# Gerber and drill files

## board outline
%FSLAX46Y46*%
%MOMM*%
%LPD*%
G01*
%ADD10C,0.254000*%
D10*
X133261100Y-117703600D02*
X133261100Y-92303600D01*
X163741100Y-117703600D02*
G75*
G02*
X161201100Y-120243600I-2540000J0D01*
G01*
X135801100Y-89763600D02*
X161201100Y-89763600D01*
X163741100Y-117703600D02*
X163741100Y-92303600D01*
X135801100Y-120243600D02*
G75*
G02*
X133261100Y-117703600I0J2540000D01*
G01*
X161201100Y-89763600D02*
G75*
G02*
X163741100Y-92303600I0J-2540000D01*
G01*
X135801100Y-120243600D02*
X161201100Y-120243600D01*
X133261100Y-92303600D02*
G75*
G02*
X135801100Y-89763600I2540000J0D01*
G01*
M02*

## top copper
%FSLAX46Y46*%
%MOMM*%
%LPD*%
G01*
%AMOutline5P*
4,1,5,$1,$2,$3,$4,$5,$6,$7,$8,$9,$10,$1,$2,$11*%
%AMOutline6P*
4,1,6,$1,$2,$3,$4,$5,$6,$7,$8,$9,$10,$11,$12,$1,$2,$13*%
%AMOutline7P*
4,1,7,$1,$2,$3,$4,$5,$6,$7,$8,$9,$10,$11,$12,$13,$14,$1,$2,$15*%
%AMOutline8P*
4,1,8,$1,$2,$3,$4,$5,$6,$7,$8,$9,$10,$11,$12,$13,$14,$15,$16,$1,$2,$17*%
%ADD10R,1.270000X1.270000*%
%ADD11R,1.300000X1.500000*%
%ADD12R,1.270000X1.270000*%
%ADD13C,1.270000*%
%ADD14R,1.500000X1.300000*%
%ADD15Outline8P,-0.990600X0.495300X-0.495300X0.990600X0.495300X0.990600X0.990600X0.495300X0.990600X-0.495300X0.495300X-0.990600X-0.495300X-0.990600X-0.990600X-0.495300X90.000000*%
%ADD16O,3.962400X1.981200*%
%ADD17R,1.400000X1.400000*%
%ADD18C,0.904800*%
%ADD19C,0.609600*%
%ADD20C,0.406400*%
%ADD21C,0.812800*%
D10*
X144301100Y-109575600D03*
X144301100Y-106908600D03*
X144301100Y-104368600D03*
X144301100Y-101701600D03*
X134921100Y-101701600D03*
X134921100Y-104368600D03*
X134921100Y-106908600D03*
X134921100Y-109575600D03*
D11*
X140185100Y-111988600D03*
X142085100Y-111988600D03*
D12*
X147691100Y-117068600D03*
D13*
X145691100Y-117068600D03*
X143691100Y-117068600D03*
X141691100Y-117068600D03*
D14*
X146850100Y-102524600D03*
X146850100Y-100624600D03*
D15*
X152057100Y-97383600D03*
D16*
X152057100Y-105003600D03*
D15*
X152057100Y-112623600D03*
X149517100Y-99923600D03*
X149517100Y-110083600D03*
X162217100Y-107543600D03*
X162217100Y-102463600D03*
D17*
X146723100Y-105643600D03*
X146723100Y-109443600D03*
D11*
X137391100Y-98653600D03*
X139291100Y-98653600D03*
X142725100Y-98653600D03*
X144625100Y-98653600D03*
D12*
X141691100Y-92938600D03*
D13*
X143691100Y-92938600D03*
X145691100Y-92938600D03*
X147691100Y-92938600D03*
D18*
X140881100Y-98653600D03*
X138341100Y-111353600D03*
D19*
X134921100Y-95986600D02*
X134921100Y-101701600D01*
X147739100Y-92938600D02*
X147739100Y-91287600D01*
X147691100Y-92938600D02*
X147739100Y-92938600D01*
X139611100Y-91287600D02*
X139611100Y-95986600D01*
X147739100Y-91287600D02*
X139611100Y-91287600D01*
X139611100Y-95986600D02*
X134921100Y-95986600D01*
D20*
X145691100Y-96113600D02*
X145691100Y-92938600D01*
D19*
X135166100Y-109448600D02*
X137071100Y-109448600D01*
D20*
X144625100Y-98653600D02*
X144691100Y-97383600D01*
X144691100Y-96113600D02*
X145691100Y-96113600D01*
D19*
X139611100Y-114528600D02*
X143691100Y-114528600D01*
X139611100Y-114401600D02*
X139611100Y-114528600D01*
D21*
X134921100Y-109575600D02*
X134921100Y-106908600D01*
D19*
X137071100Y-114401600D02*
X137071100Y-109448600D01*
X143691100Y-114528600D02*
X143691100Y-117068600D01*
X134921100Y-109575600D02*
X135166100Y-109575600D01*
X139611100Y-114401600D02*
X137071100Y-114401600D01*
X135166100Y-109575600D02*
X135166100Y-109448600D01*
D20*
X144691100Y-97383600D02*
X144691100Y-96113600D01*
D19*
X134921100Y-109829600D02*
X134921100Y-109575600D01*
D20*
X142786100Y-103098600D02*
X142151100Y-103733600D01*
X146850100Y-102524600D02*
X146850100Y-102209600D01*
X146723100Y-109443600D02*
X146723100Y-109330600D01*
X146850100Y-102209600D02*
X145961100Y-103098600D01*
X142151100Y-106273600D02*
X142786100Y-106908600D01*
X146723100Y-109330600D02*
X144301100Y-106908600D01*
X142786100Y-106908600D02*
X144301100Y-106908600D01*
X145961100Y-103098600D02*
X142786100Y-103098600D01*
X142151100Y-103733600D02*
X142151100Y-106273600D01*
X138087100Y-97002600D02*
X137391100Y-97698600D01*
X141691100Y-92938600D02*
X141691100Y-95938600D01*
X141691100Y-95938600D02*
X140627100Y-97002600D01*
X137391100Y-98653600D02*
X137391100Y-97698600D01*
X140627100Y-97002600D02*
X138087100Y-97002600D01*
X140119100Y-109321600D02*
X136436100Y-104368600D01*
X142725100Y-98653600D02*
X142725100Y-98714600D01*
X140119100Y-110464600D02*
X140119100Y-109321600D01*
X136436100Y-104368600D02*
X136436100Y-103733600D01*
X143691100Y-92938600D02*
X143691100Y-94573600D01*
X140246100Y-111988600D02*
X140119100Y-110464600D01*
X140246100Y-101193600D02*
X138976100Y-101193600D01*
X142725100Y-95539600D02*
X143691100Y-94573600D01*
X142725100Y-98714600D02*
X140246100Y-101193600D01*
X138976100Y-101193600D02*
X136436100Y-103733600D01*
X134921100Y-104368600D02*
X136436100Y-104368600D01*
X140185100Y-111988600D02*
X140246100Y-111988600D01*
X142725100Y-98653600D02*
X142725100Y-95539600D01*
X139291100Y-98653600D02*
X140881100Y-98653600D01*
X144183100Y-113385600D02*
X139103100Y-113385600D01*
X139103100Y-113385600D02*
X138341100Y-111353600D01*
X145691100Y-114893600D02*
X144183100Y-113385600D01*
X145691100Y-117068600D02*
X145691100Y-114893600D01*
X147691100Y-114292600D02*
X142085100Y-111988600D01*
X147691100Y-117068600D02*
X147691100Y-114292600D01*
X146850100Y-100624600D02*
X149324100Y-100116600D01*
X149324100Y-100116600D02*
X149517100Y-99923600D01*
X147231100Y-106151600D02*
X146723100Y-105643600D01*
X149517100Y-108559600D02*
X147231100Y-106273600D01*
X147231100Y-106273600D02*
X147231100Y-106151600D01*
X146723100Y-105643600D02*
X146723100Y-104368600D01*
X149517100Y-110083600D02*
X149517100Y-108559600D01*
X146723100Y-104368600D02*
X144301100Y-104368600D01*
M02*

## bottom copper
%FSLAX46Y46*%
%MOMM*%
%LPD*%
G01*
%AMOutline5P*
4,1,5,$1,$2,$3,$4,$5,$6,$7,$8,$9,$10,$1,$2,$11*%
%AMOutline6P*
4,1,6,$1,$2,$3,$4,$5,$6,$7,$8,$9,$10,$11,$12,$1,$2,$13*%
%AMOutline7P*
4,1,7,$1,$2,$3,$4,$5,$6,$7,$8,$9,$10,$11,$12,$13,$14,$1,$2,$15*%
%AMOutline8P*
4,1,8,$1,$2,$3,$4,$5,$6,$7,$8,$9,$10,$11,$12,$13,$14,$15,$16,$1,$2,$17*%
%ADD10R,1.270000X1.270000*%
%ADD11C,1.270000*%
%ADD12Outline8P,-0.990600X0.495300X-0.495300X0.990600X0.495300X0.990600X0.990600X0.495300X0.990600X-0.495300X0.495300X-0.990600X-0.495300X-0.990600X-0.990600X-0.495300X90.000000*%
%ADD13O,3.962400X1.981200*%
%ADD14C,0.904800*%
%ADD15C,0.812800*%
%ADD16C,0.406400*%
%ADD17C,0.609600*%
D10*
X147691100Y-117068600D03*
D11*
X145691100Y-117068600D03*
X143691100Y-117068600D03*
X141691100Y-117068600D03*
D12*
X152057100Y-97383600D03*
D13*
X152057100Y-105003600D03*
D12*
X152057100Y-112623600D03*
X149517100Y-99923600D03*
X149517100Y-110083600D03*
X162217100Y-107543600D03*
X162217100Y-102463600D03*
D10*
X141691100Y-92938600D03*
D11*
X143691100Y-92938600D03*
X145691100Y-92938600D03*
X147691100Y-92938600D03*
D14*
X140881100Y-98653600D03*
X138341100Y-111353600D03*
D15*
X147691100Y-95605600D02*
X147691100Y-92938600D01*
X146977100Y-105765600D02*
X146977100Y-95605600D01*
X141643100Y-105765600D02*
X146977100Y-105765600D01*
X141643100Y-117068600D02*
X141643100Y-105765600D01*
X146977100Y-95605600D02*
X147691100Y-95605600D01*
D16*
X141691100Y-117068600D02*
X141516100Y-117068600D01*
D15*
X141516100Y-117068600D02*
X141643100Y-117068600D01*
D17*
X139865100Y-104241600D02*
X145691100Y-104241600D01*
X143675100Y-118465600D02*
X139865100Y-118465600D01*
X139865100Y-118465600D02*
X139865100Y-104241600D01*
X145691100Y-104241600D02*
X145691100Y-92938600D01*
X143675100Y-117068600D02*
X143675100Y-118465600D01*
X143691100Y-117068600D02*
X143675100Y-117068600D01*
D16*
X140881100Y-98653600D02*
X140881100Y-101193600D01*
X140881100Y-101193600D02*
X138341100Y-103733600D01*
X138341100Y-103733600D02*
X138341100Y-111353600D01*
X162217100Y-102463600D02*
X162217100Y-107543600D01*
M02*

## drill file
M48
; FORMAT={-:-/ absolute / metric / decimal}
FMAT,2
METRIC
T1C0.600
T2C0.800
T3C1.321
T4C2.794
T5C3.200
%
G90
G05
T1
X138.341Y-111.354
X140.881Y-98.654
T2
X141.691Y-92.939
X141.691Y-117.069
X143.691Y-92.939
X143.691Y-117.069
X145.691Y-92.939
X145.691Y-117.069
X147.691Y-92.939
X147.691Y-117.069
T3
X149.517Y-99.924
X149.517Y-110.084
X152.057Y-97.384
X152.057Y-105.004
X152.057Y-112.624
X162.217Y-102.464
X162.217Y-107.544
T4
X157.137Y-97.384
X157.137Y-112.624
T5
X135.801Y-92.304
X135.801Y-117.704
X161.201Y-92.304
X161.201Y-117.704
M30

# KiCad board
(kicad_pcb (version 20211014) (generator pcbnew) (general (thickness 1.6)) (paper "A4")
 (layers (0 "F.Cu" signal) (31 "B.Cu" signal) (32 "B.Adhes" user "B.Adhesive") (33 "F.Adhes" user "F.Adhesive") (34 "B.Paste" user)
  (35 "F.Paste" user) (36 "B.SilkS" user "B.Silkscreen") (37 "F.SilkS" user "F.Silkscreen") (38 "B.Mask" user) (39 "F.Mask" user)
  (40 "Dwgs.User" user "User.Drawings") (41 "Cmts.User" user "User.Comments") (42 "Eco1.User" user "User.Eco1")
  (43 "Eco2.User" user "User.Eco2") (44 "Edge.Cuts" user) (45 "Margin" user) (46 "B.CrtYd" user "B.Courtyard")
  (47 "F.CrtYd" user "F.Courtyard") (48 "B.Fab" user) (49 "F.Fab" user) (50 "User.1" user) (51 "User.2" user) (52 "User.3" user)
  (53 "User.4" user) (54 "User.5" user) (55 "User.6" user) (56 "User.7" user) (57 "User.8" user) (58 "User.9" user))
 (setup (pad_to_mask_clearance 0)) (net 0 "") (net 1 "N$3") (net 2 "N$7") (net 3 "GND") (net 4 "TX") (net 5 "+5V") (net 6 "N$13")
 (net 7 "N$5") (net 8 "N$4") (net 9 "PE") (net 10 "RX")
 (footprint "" (layer "F.Cu") (at 135.8011 92.3036)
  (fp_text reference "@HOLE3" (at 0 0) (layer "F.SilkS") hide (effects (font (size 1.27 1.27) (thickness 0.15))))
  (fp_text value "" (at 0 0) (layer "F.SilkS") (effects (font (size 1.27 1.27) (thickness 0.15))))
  (pad "" np_thru_hole circle (at 0 0) (size 3.2 3.2) (drill 3.2) (layers *.Cu *.Mask)))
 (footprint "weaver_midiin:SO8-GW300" (layer "F.Cu") (at 139.6111 105.6386 180)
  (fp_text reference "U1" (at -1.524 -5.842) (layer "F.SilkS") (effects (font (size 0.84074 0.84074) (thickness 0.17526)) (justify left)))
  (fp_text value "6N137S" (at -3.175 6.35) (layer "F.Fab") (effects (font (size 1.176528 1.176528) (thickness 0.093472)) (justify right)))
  (pad "1" smd rect (at -4.69 -3.937 180) (size 1.27 1.27) (layers "F.Cu" "F.Paste" "F.Mask") (solder_mask_margin 0.0508))
  (pad "2" smd rect (at -4.69 -1.27 180) (size 1.27 1.27) (layers "F.Cu" "F.Paste" "F.Mask") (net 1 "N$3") (solder_mask_margin 0.0508))
  (pad "3" smd rect (at -4.69 1.27 180) (size 1.27 1.27) (layers "F.Cu" "F.Paste" "F.Mask") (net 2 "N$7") (solder_mask_margin 0.0508))
  (pad "4" smd rect (at -4.69 3.937 180) (size 1.27 1.27) (layers "F.Cu" "F.Paste" "F.Mask") (solder_mask_margin 0.0508))
  (pad "5" smd rect (at 4.69 3.937 180) (size 1.27 1.27) (layers "F.Cu" "F.Paste" "F.Mask") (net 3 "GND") (solder_mask_margin 0.0508))
  (pad "6" smd rect (at 4.69 1.27 180) (size 1.27 1.27) (layers "F.Cu" "F.Paste" "F.Mask") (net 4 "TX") (solder_mask_margin 0.0508))
  (pad "7" smd rect (at 4.69 -1.27 180) (size 1.27 1.27) (layers "F.Cu" "F.Paste" "F.Mask") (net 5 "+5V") (solder_mask_margin 0.0508))
  (pad "8" smd rect (at 4.69 -3.937 180) (size 1.27 1.27) (layers "F.Cu" "F.Paste" "F.Mask") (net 5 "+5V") (solder_mask_margin 0.0508)))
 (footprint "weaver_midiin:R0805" (layer "F.Cu") (at 141.1351 111.9886)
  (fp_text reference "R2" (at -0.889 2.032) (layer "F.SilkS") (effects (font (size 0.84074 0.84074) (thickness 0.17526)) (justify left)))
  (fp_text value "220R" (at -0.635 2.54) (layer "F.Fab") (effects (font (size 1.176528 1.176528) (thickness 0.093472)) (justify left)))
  (pad "1" smd rect (at -0.95 0) (size 1.3 1.5) (layers "F.Cu" "F.Paste" "F.Mask") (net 4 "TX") (solder_mask_margin 0.0508))
  (pad "2" smd rect (at 0.95 0) (size 1.3 1.5) (layers "F.Cu" "F.Paste" "F.Mask") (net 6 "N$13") (solder_mask_margin 0.0508)))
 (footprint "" (layer "F.Cu") (at 135.8011 117.7036)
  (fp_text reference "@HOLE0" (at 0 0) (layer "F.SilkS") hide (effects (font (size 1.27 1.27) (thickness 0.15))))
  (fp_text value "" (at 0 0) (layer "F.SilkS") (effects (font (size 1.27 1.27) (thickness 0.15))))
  (pad "" np_thru_hole circle (at 0 0) (size 3.2 3.2) (drill 3.2) (layers *.Cu *.Mask)))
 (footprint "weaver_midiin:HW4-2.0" (layer "F.Cu") (at 144.6911 117.0686 180)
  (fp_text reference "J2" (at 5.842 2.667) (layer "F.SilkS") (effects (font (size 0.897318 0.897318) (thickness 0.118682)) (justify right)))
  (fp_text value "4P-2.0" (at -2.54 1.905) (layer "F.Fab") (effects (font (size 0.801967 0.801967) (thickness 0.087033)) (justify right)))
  (pad "1" thru_hole rect (at -3 0 180) (size 1.27 1.27) (drill 0.8) (layers *.Cu *.Mask) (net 6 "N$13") (solder_mask_margin 0.0508))
  (pad "2" thru_hole circle (at -1 0 180) (size 1.27 1.27) (drill 0.8) (layers *.Cu *.Mask) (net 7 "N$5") (solder_mask_margin 0.0508))
  (pad "3" thru_hole circle (at 1 0 180) (size 1.27 1.27) (drill 0.8) (layers *.Cu *.Mask) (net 5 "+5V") (solder_mask_margin 0.0508))
  (pad "4" thru_hole circle (at 3 0 180) (size 1.27 1.27) (drill 0.8) (layers *.Cu *.Mask) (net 3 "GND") (solder_mask_margin 0.0508)))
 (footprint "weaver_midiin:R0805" (layer "F.Cu") (at 146.8501 101.5746 90)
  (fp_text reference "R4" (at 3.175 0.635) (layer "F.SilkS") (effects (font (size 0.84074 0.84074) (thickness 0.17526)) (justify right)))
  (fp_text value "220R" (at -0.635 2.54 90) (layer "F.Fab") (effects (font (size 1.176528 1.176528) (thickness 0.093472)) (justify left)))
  (pad "1" smd rect (at -0.95 0 90) (size 1.3 1.5) (layers "F.Cu" "F.Paste" "F.Mask") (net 1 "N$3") (solder_mask_margin 0.0508))
  (pad "2" smd rect (at 0.95 0 90) (size 1.3 1.5) (layers "F.Cu" "F.Paste" "F.Mask") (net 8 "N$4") (solder_mask_margin 0.0508)))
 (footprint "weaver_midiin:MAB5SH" (layer "F.Cu") (at 157.1371 105.0036 90)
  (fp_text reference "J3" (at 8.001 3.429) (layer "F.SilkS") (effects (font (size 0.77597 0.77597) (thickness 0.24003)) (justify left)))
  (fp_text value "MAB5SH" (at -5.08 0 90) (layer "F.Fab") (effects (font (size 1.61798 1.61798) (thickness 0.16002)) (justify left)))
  (pad "" np_thru_hole circle (at 7.62 0 90) (size 2.794 2.794) (drill 2.794) (layers *.Cu *.Mask))
  (pad "" np_thru_hole circle (at -7.62 0 90) (size 2.794 2.794) (drill 2.794) (layers *.Cu *.Mask))
  (pad "1" thru_hole roundrect (at 7.62 -5.08 90) (size 1.9812 1.9812) (drill 1.3208) (layers *.Cu *.Mask) (roundrect_rratio 0.25)
   (chamfer_ratio 0.25) (chamfer top_left top_right bottom_left bottom_right) (solder_mask_margin 0.0508))
  (pad "2" thru_hole oval (at 0 -5.08 180) (size 3.9624 1.9812) (drill 1.3208) (layers *.Cu *.Mask) (solder_mask_margin 0.0508))
  (pad "3" thru_hole roundrect (at -7.62 -5.08 90) (size 1.9812 1.9812) (drill 1.3208) (layers *.Cu *.Mask) (roundrect_rratio 0.25)
   (chamfer_ratio 0.25) (chamfer top_left top_right bottom_left bottom_right) (solder_mask_margin 0.0508))
  (pad "4" thru_hole roundrect (at 5.08 -7.62 90) (size 1.9812 1.9812) (drill 1.3208) (layers *.Cu *.Mask) (roundrect_rratio 0.25)
   (chamfer_ratio 0.25) (chamfer top_left top_right bottom_left bottom_right) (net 8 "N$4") (solder_mask_margin 0.0508))
  (pad "5" thru_hole roundrect (at -5.08 -7.62 90) (size 1.9812 1.9812) (drill 1.3208) (layers *.Cu *.Mask) (roundrect_rratio 0.25)
   (chamfer_ratio 0.25) (chamfer top_left top_right bottom_left bottom_right) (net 2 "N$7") (solder_mask_margin 0.0508))
  (pad "PE" thru_hole roundrect (at -2.54 5.08 90) (size 1.9812 1.9812) (drill 1.3208) (layers *.Cu *.Mask) (roundrect_rratio 0.25)
   (chamfer_ratio 0.25) (chamfer top_left top_right bottom_left bottom_right) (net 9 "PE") (solder_mask_margin 0.0508))
  (pad "PE@" thru_hole roundrect (at 2.54 5.08 90) (size 1.9812 1.9812) (drill 1.3208) (layers *.Cu *.Mask) (roundrect_rratio 0.25)
   (chamfer_ratio 0.25) (chamfer top_left top_right bottom_left bottom_right) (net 9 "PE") (solder_mask_margin 0.0508)))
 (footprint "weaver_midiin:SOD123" (layer "F.Cu") (at 146.7231 107.5436 90)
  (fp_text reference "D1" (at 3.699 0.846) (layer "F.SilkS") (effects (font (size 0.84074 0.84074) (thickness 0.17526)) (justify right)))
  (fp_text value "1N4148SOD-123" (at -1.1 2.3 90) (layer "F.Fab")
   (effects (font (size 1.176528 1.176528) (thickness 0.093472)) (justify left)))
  (pad "A" smd rect (at 1.9 0 90) (size 1.4 1.4) (layers "F.Cu" "F.Paste" "F.Mask") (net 2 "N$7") (solder_mask_margin 0.0508))
  (pad "C" smd rect (at -1.9 0 90) (size 1.4 1.4) (layers "F.Cu" "F.Paste" "F.Mask") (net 1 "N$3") (solder_mask_margin 0.0508)))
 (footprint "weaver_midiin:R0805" (layer "F.Cu") (at 138.3411 98.6536)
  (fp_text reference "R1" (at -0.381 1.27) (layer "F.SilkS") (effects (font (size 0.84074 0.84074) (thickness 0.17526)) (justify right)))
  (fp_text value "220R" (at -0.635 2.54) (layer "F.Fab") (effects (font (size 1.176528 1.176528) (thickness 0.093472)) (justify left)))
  (pad "1" smd rect (at -0.95 0) (size 1.3 1.5) (layers "F.Cu" "F.Paste" "F.Mask") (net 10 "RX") (solder_mask_margin 0.0508))
  (pad "2" smd rect (at 0.95 0) (size 1.3 1.5) (layers "F.Cu" "F.Paste" "F.Mask") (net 7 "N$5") (solder_mask_margin 0.0508)))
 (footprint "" (layer "F.Cu") (at 161.2011 117.7036)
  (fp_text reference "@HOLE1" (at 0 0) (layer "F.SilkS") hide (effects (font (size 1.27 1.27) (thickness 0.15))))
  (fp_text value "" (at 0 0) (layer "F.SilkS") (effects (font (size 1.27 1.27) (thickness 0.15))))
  (pad "" np_thru_hole circle (at 0 0) (size 3.2 3.2) (drill 3.2) (layers *.Cu *.Mask)))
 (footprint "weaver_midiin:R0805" (layer "F.Cu") (at 143.6751 98.6536)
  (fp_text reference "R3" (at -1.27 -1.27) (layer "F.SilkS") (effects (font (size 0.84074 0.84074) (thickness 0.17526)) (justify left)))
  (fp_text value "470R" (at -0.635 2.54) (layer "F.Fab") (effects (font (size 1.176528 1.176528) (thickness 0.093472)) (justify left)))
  (pad "1" smd rect (at -0.95 0) (size 1.3 1.5) (layers "F.Cu" "F.Paste" "F.Mask") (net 4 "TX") (solder_mask_margin 0.0508))
  (pad "2" smd rect (at 0.95 0) (size 1.3 1.5) (layers "F.Cu" "F.Paste" "F.Mask") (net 5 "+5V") (solder_mask_margin 0.0508)))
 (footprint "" (layer "F.Cu") (at 161.2011 92.3036)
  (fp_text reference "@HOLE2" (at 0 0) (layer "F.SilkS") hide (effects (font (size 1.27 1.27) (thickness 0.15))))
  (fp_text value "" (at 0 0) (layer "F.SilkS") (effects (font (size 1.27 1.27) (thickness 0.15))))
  (pad "" np_thru_hole circle (at 0 0) (size 3.2 3.2) (drill 3.2) (layers *.Cu *.Mask)))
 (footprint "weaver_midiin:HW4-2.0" (layer "F.Cu") (at 144.6911 92.9386)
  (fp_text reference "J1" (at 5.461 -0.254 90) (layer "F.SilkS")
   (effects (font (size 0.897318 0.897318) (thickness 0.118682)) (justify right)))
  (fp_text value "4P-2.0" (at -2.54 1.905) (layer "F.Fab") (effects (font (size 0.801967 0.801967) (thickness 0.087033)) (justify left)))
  (pad "1" thru_hole rect (at -3 0) (size 1.27 1.27) (drill 0.8) (layers *.Cu *.Mask) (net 10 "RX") (solder_mask_margin 0.0508))
  (pad "2" thru_hole circle (at -1 0) (size 1.27 1.27) (drill 0.8) (layers *.Cu *.Mask) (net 4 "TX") (solder_mask_margin 0.0508))
  (pad "3" thru_hole circle (at 1 0) (size 1.27 1.27) (drill 0.8) (layers *.Cu *.Mask) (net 5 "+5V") (solder_mask_margin 0.0508))
  (pad "4" thru_hole circle (at 3 0) (size 1.27 1.27) (drill 0.8) (layers *.Cu *.Mask) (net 3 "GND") (solder_mask_margin 0.0508)))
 (gr_line (start 133.2611 117.7036) (end 133.2611 92.3036) (layer "Edge.Cuts") (width 0.254))
 (gr_arc (start 163.7411 117.7036) (mid 162.997151 119.499651) (end 161.2011 120.2436) (layer "Edge.Cuts") (width 0.254))
 (gr_line (start 135.8011 89.7636) (end 161.2011 89.7636) (layer "Edge.Cuts") (width 0.254))
 (gr_line (start 163.7411 117.7036) (end 163.7411 92.3036) (layer "Edge.Cuts") (width 0.254))
 (gr_arc (start 135.8011 120.2436) (mid 134.005049 119.499651) (end 133.2611 117.7036) (layer "Edge.Cuts") (width 0.254))
 (gr_arc (start 161.2011 89.7636) (mid 162.997151 90.507549) (end 163.7411 92.3036) (layer "Edge.Cuts") (width 0.254))
 (gr_line (start 135.8011 120.2436) (end 161.2011 120.2436) (layer "Edge.Cuts") (width 0.254))
 (gr_arc (start 133.2611 92.3036) (mid 134.005049 90.507549) (end 135.8011 89.7636) (layer "Edge.Cuts") (width 0.254))
 (segment (start 134.9211 95.9866) (end 134.9211 101.7016) (width 0.6096) (layer "F.Cu") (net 3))
 (segment (start 147.7391 92.9386) (end 147.7391 91.2876) (width 0.6096) (layer "F.Cu") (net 3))
 (segment (start 147.6911 92.9386) (end 147.7391 92.9386) (width 0.6096) (layer "F.Cu") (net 3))
 (segment (start 139.6111 91.2876) (end 139.6111 95.9866) (width 0.6096) (layer "F.Cu") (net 3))
 (segment (start 147.7391 91.2876) (end 139.6111 91.2876) (width 0.6096) (layer "F.Cu") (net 3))
 (segment (start 139.6111 95.9866) (end 134.9211 95.9866) (width 0.6096) (layer "F.Cu") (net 3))
 (segment (start 147.6911 95.6056) (end 147.6911 92.9386) (width 0.8128) (layer "B.Cu") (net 3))
 (segment (start 146.9771 105.7656) (end 146.9771 95.6056) (width 0.8128) (layer "B.Cu") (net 3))
 (segment (start 141.6431 105.7656) (end 146.9771 105.7656) (width 0.8128) (layer "B.Cu") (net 3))
 (segment (start 141.6431 117.0686) (end 141.6431 105.7656) (width 0.8128) (layer "B.Cu") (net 3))
 (segment (start 146.9771 95.6056) (end 147.6911 95.6056) (width 0.8128) (layer "B.Cu") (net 3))
 (segment (start 141.6911 117.0686) (end 141.5161 117.0686) (width 0.4064) (layer "B.Cu") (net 3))
 (segment (start 141.5161 117.0686) (end 141.6431 117.0686) (width 0.8128) (layer "B.Cu") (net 3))
 (segment (start 145.6911 96.1136) (end 145.6911 92.9386) (width 0.4064) (layer "F.Cu") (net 5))
 (segment (start 135.1661 109.4486) (end 137.0711 109.4486) (width 0.6096) (layer "F.Cu") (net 5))
 (segment (start 144.6251 98.6536) (end 144.6911 97.3836) (width 0.4064) (layer "F.Cu") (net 5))
 (segment (start 144.6911 96.1136) (end 145.6911 96.1136) (width 0.4064) (layer "F.Cu") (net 5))
 (segment (start 139.6111 114.5286) (end 143.6911 114.5286) (width 0.6096) (layer "F.Cu") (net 5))
 (segment (start 139.6111 114.4016) (end 139.6111 114.5286) (width 0.6096) (layer "F.Cu") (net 5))
 (segment (start 134.9211 109.5756) (end 134.9211 106.9086) (width 0.8128) (layer "F.Cu") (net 5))
 (segment (start 137.0711 114.4016) (end 137.0711 109.4486) (width 0.6096) (layer "F.Cu") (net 5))
 (segment (start 143.6911 114.5286) (end 143.6911 117.0686) (width 0.6096) (layer "F.Cu") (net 5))
 (segment (start 134.9211 109.5756) (end 135.1661 109.5756) (width 0.6096) (layer "F.Cu") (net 5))
 (segment (start 139.6111 114.4016) (end 137.0711 114.4016) (width 0.6096) (layer "F.Cu") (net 5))
 (segment (start 135.1661 109.5756) (end 135.1661 109.4486) (width 0.6096) (layer "F.Cu") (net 5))
 (segment (start 144.6911 97.3836) (end 144.6911 96.1136) (width 0.4064) (layer "F.Cu") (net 5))
 (segment (start 134.9211 109.8296) (end 134.9211 109.5756) (width 0.6096) (layer "F.Cu") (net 5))
 (segment (start 139.8651 104.2416) (end 145.6911 104.2416) (width 0.6096) (layer "B.Cu") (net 5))
 (segment (start 143.6751 118.4656) (end 139.8651 118.4656) (width 0.6096) (layer "B.Cu") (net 5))
 (segment (start 139.8651 118.4656) (end 139.8651 104.2416) (width 0.6096) (layer "B.Cu") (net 5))
 (segment (start 145.6911 104.2416) (end 145.6911 92.9386) (width 0.6096) (layer "B.Cu") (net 5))
 (segment (start 143.6751 117.0686) (end 143.6751 118.4656) (width 0.6096) (layer "B.Cu") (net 5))
 (segment (start 143.6911 117.0686) (end 143.6751 117.0686) (width 0.6096) (layer "B.Cu") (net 5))
 (segment (start 142.7861 103.0986) (end 142.1511 103.7336) (width 0.4064) (layer "F.Cu") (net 1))
 (segment (start 146.8501 102.5246) (end 146.8501 102.2096) (width 0.4064) (layer "F.Cu") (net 1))
 (segment (start 146.7231 109.4436) (end 146.7231 109.3306) (width 0.4064) (layer "F.Cu") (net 1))
 (segment (start 146.8501 102.2096) (end 145.9611 103.0986) (width 0.4064) (layer "F.Cu") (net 1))
 (segment (start 142.1511 106.2736) (end 142.7861 106.9086) (width 0.4064) (layer "F.Cu") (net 1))
 (segment (start 146.7231 109.3306) (end 144.3011 106.9086) (width 0.4064) (layer "F.Cu") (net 1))
 (segment (start 142.7861 106.9086) (end 144.3011 106.9086) (width 0.4064) (layer "F.Cu") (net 1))
 (segment (start 145.9611 103.0986) (end 142.7861 103.0986) (width 0.4064) (layer "F.Cu") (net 1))
 (segment (start 142.1511 103.7336) (end 142.1511 106.2736) (width 0.4064) (layer "F.Cu") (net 1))
 (segment (start 138.0871 97.0026) (end 137.3911 97.6986) (width 0.4064) (layer "F.Cu") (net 10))
 (segment (start 141.6911 92.9386) (end 141.6911 95.9386) (width 0.4064) (layer "F.Cu") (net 10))
 (segment (start 141.6911 95.9386) (end 140.6271 97.0026) (width 0.4064) (layer "F.Cu") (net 10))
 (segment (start 137.3911 98.6536) (end 137.3911 97.6986) (width 0.4064) (layer "F.Cu") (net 10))
 (segment (start 140.6271 97.0026) (end 138.0871 97.0026) (width 0.4064) (layer "F.Cu") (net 10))
 (segment (start 140.1191 109.3216) (end 136.4361 104.3686) (width 0.4064) (layer "F.Cu") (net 4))
 (segment (start 142.7251 98.6536) (end 142.7251 98.7146) (width 0.4064) (layer "F.Cu") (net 4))
 (segment (start 140.1191 110.4646) (end 140.1191 109.3216) (width 0.4064) (layer "F.Cu") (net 4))
 (segment (start 136.4361 104.3686) (end 136.4361 103.7336) (width 0.4064) (layer "F.Cu") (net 4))
 (segment (start 143.6911 92.9386) (end 143.6911 94.5736) (width 0.4064) (layer "F.Cu") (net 4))
 (segment (start 140.2461 111.9886) (end 140.1191 110.4646) (width 0.4064) (layer "F.Cu") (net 4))
 (segment (start 140.2461 101.1936) (end 138.9761 101.1936) (width 0.4064) (layer "F.Cu") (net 4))
 (segment (start 142.7251 95.5396) (end 143.6911 94.5736) (width 0.4064) (layer "F.Cu") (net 4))
 (segment (start 142.7251 98.7146) (end 140.2461 101.1936) (width 0.4064) (layer "F.Cu") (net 4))
 (segment (start 138.9761 101.1936) (end 136.4361 103.7336) (width 0.4064) (layer "F.Cu") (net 4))
 (segment (start 134.9211 104.3686) (end 136.4361 104.3686) (width 0.4064) (layer "F.Cu") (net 4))
 (segment (start 140.1851 111.9886) (end 140.2461 111.9886) (width 0.4064) (layer "F.Cu") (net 4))
 (segment (start 142.7251 98.6536) (end 142.7251 95.5396) (width 0.4064) (layer "F.Cu") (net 4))
 (segment (start 139.2911 98.6536) (end 140.8811 98.6536) (width 0.4064) (layer "F.Cu") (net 7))
 (segment (start 144.1831 113.3856) (end 139.1031 113.3856) (width 0.4064) (layer "F.Cu") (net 7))
 (segment (start 139.1031 113.3856) (end 138.3411 111.3536) (width 0.4064) (layer "F.Cu") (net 7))
 (segment (start 145.6911 114.8936) (end 144.1831 113.3856) (width 0.4064) (layer "F.Cu") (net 7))
 (segment (start 145.6911 117.0686) (end 145.6911 114.8936) (width 0.4064) (layer "F.Cu") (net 7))
 (via (at 140.8811 98.6536) (size 0.9048) (drill 0.6) (layers "F.Cu" "B.Cu") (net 7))
 (via (at 138.3411 111.3536) (size 0.9048) (drill 0.6) (layers "F.Cu" "B.Cu") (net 7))
 (segment (start 140.8811 98.6536) (end 140.8811 101.1936) (width 0.4064) (layer "B.Cu") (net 7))
 (segment (start 140.8811 101.1936) (end 138.3411 103.7336) (width 0.4064) (layer "B.Cu") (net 7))
 (segment (start 138.3411 103.7336) (end 138.3411 111.3536) (width 0.4064) (layer "B.Cu") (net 7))
 (segment (start 147.6911 114.2926) (end 142.0851 111.9886) (width 0.4064) (layer "F.Cu") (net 6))
 (segment (start 147.6911 117.0686) (end 147.6911 114.2926) (width 0.4064) (layer "F.Cu") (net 6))
 (segment (start 146.8501 100.6246) (end 149.3241 100.1166) (width 0.4064) (layer "F.Cu") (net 8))
 (segment (start 149.3241 100.1166) (end 149.5171 99.9236) (width 0.4064) (layer "F.Cu") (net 8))
 (segment (start 147.2311 106.1516) (end 146.7231 105.6436) (width 0.4064) (layer "F.Cu") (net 2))
 (segment (start 149.5171 108.5596) (end 147.2311 106.2736) (width 0.4064) (layer "F.Cu") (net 2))
 (segment (start 147.2311 106.2736) (end 147.2311 106.1516) (width 0.4064) (layer "F.Cu") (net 2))
 (segment (start 146.7231 105.6436) (end 146.7231 104.3686) (width 0.4064) (layer "F.Cu") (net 2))
 (segment (start 149.5171 110.0836) (end 149.5171 108.5596) (width 0.4064) (layer "F.Cu") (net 2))
 (segment (start 146.7231 104.3686) (end 144.3011 104.3686) (width 0.4064) (layer "F.Cu") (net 2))
 (segment (start 162.2171 102.4636) (end 162.2171 107.5436) (width 0.4064) (layer "B.Cu") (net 9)))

